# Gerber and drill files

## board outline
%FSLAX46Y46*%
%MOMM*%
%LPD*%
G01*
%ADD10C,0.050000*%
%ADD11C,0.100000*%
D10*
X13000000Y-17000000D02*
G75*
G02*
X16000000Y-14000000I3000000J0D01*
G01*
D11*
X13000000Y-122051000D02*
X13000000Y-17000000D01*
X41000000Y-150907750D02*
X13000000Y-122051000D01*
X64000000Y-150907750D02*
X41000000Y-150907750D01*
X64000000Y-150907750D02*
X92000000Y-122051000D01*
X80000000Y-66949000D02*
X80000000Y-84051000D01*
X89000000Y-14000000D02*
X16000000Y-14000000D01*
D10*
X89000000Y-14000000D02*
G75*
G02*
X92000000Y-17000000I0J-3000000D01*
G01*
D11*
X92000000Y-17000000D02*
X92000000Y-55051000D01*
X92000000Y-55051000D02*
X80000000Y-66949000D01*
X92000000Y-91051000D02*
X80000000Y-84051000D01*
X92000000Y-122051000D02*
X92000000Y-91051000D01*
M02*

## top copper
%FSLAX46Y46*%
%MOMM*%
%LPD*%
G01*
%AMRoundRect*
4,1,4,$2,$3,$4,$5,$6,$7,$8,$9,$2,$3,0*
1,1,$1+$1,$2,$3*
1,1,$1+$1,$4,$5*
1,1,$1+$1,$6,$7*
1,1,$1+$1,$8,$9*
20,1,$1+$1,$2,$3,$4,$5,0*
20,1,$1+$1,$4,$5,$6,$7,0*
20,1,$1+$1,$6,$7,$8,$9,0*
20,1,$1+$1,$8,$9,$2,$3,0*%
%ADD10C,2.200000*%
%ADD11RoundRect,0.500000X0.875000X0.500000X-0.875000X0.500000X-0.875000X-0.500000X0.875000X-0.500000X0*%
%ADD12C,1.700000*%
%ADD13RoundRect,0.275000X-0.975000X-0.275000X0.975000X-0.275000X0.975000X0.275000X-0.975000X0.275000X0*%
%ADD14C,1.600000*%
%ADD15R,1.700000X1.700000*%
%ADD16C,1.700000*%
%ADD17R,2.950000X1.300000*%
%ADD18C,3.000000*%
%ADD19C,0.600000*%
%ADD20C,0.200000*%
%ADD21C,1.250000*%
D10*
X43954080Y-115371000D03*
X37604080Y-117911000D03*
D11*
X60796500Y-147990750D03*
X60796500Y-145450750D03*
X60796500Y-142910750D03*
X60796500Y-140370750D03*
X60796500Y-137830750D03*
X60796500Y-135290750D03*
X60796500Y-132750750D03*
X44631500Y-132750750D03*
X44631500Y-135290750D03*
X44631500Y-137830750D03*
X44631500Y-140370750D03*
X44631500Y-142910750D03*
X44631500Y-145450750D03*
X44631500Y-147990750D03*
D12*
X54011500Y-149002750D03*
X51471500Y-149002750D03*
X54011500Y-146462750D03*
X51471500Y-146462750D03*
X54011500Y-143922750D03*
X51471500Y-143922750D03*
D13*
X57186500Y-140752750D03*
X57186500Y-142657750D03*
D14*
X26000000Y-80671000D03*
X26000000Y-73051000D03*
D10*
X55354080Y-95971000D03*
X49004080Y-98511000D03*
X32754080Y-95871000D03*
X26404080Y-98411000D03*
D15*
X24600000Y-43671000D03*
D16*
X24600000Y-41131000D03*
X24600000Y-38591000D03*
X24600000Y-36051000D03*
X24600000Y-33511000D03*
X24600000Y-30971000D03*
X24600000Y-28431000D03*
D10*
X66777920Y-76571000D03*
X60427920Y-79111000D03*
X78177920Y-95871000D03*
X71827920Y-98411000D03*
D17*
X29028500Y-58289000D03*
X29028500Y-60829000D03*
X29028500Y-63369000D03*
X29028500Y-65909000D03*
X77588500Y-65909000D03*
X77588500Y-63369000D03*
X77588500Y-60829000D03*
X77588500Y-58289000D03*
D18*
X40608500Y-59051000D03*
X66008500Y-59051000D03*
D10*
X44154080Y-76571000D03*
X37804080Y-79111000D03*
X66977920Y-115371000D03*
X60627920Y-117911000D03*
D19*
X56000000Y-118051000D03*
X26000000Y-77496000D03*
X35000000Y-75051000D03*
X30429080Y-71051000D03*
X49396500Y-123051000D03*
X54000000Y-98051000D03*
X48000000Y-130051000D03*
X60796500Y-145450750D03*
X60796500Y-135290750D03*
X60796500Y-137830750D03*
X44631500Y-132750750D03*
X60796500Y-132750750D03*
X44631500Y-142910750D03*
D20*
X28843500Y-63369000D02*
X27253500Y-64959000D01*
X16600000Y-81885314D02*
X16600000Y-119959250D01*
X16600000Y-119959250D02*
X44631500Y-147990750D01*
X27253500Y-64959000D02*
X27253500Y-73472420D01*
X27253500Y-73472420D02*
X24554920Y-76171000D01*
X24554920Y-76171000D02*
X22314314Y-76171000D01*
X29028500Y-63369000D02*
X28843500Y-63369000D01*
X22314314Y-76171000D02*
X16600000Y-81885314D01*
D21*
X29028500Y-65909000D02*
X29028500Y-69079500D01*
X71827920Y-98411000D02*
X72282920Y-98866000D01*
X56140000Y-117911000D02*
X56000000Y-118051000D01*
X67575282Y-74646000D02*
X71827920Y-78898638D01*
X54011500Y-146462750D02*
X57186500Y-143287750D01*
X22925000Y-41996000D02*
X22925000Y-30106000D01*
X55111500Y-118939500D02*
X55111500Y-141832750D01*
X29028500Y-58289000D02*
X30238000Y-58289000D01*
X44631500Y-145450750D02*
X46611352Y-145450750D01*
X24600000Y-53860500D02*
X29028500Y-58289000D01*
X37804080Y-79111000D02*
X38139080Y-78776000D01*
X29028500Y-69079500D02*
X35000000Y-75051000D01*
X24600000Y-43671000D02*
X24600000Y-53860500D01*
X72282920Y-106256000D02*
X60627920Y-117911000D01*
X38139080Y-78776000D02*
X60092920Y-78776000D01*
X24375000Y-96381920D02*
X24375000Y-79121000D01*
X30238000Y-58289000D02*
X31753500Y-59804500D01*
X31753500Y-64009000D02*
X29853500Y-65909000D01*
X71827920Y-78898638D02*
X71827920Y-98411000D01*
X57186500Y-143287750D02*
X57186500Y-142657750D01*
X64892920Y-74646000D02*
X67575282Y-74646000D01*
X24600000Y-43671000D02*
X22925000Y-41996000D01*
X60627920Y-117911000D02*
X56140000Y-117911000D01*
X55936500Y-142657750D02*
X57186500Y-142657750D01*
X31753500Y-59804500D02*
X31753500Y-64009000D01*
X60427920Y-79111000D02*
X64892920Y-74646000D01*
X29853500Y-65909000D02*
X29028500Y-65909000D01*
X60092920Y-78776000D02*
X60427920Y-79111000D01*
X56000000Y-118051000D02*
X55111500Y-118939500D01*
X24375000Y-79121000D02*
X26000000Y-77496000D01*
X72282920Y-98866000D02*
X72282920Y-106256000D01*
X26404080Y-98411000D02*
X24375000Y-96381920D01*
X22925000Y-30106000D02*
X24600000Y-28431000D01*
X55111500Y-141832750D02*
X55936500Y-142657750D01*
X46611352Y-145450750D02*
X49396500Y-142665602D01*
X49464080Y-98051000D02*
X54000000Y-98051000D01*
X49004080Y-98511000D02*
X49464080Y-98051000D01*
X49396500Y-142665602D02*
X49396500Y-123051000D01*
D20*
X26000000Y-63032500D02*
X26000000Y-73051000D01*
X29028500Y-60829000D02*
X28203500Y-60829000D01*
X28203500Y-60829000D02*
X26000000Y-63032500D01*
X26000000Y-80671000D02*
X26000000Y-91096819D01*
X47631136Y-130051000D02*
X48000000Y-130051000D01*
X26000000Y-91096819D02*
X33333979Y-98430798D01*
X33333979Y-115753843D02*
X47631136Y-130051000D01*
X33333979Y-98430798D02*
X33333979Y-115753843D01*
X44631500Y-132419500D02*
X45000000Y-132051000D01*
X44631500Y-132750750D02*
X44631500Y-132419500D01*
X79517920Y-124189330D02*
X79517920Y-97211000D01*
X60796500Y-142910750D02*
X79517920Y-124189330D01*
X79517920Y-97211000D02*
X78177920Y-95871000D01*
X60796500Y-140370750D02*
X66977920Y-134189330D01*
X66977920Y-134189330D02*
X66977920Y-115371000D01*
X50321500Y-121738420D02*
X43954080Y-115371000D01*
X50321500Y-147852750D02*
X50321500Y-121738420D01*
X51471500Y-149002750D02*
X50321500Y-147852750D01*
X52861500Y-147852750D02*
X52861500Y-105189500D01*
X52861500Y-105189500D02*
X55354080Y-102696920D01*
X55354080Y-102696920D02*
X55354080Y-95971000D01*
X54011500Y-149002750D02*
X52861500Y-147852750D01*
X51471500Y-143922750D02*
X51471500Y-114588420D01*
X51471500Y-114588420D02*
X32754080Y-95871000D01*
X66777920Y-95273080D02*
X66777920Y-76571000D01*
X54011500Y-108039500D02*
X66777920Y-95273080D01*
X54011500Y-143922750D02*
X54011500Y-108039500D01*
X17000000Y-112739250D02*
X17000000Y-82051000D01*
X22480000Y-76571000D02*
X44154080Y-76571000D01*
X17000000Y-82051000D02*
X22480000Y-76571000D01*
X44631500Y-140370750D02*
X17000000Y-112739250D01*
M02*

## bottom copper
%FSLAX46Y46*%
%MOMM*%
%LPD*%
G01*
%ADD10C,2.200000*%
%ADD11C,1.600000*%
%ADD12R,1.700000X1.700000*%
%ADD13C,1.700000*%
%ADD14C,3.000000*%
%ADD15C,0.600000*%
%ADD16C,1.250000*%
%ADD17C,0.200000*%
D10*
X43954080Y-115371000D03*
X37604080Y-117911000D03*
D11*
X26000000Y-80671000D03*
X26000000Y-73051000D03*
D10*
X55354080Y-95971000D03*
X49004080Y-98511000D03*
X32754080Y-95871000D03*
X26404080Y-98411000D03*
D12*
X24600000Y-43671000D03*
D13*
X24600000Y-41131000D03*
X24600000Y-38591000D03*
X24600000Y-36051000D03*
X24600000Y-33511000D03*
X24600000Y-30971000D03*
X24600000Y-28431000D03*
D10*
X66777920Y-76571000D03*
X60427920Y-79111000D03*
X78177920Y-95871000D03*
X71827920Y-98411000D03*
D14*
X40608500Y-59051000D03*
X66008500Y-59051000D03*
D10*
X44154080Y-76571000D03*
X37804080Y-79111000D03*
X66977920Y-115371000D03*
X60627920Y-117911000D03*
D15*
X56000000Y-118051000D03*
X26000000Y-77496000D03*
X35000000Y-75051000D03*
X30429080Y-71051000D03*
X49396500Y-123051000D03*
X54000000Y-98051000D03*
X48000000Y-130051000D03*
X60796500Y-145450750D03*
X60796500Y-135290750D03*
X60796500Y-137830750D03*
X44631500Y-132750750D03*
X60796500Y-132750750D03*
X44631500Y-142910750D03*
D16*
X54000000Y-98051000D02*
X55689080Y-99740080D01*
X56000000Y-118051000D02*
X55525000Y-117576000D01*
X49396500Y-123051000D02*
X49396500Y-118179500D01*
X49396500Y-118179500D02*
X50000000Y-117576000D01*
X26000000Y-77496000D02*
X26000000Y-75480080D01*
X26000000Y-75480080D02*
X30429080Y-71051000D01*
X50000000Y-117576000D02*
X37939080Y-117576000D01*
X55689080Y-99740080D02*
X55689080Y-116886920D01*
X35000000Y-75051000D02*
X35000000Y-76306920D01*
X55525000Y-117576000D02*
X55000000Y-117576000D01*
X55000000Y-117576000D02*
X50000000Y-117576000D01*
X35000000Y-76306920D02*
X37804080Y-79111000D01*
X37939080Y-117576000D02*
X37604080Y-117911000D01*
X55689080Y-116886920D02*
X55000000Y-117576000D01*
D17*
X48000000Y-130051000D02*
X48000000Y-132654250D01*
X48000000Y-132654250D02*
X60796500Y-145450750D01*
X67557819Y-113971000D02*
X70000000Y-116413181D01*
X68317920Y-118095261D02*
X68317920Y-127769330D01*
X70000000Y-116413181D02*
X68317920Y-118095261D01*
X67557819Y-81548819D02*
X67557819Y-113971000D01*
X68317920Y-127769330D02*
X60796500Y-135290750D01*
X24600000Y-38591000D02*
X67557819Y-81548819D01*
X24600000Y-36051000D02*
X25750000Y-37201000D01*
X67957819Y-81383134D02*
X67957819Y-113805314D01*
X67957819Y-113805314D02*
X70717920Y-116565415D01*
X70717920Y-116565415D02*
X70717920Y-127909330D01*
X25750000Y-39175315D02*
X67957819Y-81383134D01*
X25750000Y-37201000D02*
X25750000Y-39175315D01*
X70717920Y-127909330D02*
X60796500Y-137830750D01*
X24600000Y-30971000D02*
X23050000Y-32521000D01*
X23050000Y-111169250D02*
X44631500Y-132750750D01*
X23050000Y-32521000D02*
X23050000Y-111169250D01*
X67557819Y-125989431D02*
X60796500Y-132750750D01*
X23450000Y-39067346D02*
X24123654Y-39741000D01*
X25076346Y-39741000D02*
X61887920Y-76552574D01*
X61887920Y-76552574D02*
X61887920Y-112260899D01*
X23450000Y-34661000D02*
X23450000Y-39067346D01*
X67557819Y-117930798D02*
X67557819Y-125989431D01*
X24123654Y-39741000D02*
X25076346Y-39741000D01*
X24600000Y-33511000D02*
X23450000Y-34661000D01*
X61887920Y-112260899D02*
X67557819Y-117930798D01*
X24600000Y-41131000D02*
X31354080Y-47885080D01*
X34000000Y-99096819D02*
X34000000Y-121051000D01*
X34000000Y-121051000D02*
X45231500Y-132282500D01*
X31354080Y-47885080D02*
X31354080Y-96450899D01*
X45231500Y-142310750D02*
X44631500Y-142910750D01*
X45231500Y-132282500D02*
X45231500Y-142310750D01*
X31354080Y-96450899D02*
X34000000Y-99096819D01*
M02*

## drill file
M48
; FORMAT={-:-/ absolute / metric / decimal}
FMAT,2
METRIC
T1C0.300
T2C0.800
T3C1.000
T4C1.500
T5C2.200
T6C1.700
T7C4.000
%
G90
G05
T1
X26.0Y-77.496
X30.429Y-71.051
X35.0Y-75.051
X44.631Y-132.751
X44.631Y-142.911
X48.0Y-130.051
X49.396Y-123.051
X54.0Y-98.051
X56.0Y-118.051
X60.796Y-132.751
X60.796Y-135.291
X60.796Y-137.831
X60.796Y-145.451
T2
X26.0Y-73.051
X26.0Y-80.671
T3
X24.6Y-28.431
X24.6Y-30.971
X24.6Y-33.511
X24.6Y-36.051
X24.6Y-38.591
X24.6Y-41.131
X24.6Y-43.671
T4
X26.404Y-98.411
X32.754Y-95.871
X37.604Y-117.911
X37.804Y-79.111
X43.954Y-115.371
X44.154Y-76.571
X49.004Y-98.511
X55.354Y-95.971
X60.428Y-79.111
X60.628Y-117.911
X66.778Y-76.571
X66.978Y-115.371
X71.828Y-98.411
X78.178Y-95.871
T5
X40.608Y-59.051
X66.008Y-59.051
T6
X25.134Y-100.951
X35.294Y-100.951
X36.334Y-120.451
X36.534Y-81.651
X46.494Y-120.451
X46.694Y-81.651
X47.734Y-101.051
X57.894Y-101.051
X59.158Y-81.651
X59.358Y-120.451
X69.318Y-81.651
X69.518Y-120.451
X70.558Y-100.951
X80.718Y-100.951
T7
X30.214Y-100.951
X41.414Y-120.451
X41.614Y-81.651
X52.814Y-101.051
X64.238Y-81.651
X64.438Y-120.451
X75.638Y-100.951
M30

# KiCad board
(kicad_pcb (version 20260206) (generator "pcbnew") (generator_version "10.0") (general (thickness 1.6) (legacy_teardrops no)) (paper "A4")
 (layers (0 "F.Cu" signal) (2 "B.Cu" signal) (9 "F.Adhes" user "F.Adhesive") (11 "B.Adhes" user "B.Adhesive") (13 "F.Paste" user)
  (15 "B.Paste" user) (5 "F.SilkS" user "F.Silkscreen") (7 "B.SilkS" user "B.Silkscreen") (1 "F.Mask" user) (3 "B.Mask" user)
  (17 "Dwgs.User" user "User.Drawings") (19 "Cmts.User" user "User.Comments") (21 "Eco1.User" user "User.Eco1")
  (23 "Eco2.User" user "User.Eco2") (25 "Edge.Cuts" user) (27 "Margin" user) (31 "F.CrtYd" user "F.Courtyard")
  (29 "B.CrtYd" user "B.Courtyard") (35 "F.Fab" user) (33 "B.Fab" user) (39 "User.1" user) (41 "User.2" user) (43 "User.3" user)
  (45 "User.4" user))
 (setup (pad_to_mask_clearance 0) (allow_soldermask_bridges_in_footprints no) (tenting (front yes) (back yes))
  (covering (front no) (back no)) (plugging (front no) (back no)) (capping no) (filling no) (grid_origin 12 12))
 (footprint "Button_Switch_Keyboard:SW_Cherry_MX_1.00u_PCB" (layer "F.Cu") (at 43.95408 115.371)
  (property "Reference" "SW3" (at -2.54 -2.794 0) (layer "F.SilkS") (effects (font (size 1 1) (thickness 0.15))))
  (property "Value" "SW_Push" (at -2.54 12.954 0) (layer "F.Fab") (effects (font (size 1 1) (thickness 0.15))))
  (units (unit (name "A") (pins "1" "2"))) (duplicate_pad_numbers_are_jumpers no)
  (pad "" np_thru_hole circle (at -7.62 5.08) (size 1.7 1.7) (drill 1.7) (layers "*.Cu" "*.Mask"))
  (pad "" np_thru_hole circle (at -2.54 5.08) (size 4 4) (drill 4) (layers "*.Cu" "*.Mask"))
  (pad "" np_thru_hole circle (at 2.54 5.08) (size 1.7 1.7) (drill 1.7) (layers "*.Cu" "*.Mask"))
  (pad "1" thru_hole circle (at 0 0) (size 2.2 2.2) (drill 1.5) (layers "*.Cu" "*.Mask") (remove_unused_layers no) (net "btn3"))
  (pad "2" thru_hole circle (at -6.35 2.54) (size 2.2 2.2) (drill 1.5) (layers "*.Cu" "*.Mask") (remove_unused_layers no) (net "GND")))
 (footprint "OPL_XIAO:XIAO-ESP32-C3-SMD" (layer "F.Cu") (at 61.6315 129.87075 180)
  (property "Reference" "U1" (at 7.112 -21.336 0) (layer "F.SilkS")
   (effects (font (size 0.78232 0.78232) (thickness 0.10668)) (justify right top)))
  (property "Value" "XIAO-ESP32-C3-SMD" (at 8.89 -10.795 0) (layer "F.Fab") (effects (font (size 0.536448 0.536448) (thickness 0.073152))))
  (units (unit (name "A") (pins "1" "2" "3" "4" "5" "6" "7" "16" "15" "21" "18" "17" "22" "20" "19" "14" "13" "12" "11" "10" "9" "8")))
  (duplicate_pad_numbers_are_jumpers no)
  (pad "1" smd roundrect (at 0.835 -18.12 180) (size 2.75 2) (layers "F.Cu" "F.Mask" "F.Paste") (roundrect_rratio 0.25)
   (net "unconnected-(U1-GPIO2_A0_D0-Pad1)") (solder_mask_margin 0.0508) (thermal_bridge_angle 45))
  (pad "2" smd roundrect (at 0.835 -15.58 180) (size 2.75 2) (layers "F.Cu" "F.Mask" "F.Paste") (roundrect_rratio 0.25) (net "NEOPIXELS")
   (solder_mask_margin 0.0508) (thermal_bridge_angle 45))
  (pad "3" smd roundrect (at 0.835 -13.04 180) (size 2.75 2) (layers "F.Cu" "F.Mask" "F.Paste") (roundrect_rratio 0.25) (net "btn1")
   (solder_mask_margin 0.0508) (thermal_bridge_angle 45))
  (pad "4" smd roundrect (at 0.835 -10.5 180) (size 2.75 2) (layers "F.Cu" "F.Mask" "F.Paste") (roundrect_rratio 0.25) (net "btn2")
   (solder_mask_margin 0.0508) (thermal_bridge_angle 45))
  (pad "5" smd roundrect (at 0.835 -7.96 180) (size 2.75 2) (layers "F.Cu" "F.Mask" "F.Paste") (roundrect_rratio 0.25) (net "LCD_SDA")
   (solder_mask_margin 0.0508) (thermal_bridge_angle 45))
  (pad "6" smd roundrect (at 0.835 -5.42 180) (size 2.75 2) (layers "F.Cu" "F.Mask" "F.Paste") (roundrect_rratio 0.25) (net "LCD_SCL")
   (solder_mask_margin 0.0508) (thermal_bridge_angle 45))
  (pad "7" smd roundrect (at 0.835 -2.88 180) (size 2.75 2) (layers "F.Cu" "F.Mask" "F.Paste") (roundrect_rratio 0.25) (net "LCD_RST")
   (solder_mask_margin 0.0508) (thermal_bridge_angle 45))
  (pad "8" smd roundrect (at 17 -2.88 180) (size 2.75 2) (layers "F.Cu" "F.Mask" "F.Paste") (roundrect_rratio 0.25) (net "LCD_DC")
   (solder_mask_margin 0.0508) (thermal_bridge_angle 45))
  (pad "9" smd roundrect (at 17 -5.42 180) (size 2.75 2) (layers "F.Cu" "F.Mask" "F.Paste") (roundrect_rratio 0.25)
   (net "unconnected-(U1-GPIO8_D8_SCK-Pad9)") (solder_mask_margin 0.0508) (thermal_bridge_angle 45))
  (pad "10" smd roundrect (at 17 -7.96 180) (size 2.75 2) (layers "F.Cu" "F.Mask" "F.Paste") (roundrect_rratio 0.25)
   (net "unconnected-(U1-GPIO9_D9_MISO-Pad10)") (solder_mask_margin 0.0508) (thermal_bridge_angle 45))
  (pad "11" smd roundrect (at 17 -10.5 180) (size 2.75 2) (layers "F.Cu" "F.Mask" "F.Paste") (roundrect_rratio 0.25) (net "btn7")
   (solder_mask_margin 0.0508) (thermal_bridge_angle 45))
  (pad "12" smd roundrect (at 17 -13.04 180) (size 2.75 2) (layers "F.Cu" "F.Mask" "F.Paste") (roundrect_rratio 0.25) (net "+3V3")
   (solder_mask_margin 0.0508) (thermal_bridge_angle 45))
  (pad "13" smd roundrect (at 17 -15.58 180) (size 2.75 2) (layers "F.Cu" "F.Mask" "F.Paste") (roundrect_rratio 0.25) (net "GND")
   (solder_mask_margin 0.0508) (thermal_bridge_angle 45))
  (pad "14" smd roundrect (at 17 -18.12 180) (size 2.75 2) (layers "F.Cu" "F.Mask" "F.Paste") (roundrect_rratio 0.25) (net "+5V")
   (solder_mask_margin 0.0508) (thermal_bridge_angle 45))
  (pad "15" smd circle (at 7.62 -19.132 180) (size 1.7 1.7) (layers "F.Cu" "F.Mask" "F.Paste") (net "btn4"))
  (pad "16" smd circle (at 10.16 -19.132 180) (size 1.7 1.7) (layers "F.Cu" "F.Mask" "F.Paste") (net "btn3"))
  (pad "17" smd circle (at 7.62 -16.592 180) (size 1.7 1.7) (layers "F.Cu" "F.Mask" "F.Paste") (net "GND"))
  (pad "18" smd circle (at 10.16 -16.592 180) (size 1.7 1.7) (layers "F.Cu" "F.Mask" "F.Paste") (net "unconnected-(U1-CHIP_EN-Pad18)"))
  (pad "19" smd circle (at 7.62 -14.052 180) (size 1.7 1.7) (layers "F.Cu" "F.Mask" "F.Paste") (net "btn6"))
  (pad "20" smd circle (at 10.16 -14.052 180) (size 1.7 1.7) (layers "F.Cu" "F.Mask" "F.Paste") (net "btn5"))
  (pad "21" smd roundrect (at 4.445 -10.882) (size 2.5 1.1) (layers "F.Cu" "F.Mask" "F.Paste") (roundrect_rratio 0.25) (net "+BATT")
   (thermal_bridge_angle 45))
  (pad "22" smd roundrect (at 4.445 -12.787) (size 2.5 1.1) (layers "F.Cu" "F.Mask" "F.Paste") (roundrect_rratio 0.25) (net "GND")
   (thermal_bridge_angle 45)))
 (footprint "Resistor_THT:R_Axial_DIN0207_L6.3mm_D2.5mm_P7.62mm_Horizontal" (layer "F.Cu") (at 26 80.671 90)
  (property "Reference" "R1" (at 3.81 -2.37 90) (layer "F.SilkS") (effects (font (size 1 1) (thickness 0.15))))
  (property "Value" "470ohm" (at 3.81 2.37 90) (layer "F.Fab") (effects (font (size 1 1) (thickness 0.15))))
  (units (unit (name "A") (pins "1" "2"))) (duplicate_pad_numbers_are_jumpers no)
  (pad "1" thru_hole circle (at 0 0 90) (size 1.6 1.6) (drill 0.8) (layers "*.Cu" "*.Mask") (remove_unused_layers no) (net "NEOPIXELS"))
  (pad "2" thru_hole circle (at 7.62 0 90) (size 1.6 1.6) (drill 0.8) (layers "*.Cu" "*.Mask") (remove_unused_layers no)
   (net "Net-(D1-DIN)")))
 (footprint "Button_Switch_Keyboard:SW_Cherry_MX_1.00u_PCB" (layer "F.Cu") (at 55.35408 95.971)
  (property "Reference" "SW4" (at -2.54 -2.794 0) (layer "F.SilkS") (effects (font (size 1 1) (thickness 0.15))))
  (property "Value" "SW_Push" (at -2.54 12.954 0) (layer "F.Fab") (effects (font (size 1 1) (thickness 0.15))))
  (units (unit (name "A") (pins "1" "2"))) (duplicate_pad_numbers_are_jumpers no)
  (pad "" np_thru_hole circle (at -7.62 5.08) (size 1.7 1.7) (drill 1.7) (layers "*.Cu" "*.Mask"))
  (pad "" np_thru_hole circle (at -2.54 5.08) (size 4 4) (drill 4) (layers "*.Cu" "*.Mask"))
  (pad "" np_thru_hole circle (at 2.54 5.08) (size 1.7 1.7) (drill 1.7) (layers "*.Cu" "*.Mask"))
  (pad "1" thru_hole circle (at 0 0) (size 2.2 2.2) (drill 1.5) (layers "*.Cu" "*.Mask") (remove_unused_layers no) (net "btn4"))
  (pad "2" thru_hole circle (at -6.35 2.54) (size 2.2 2.2) (drill 1.5) (layers "*.Cu" "*.Mask") (remove_unused_layers no) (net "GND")))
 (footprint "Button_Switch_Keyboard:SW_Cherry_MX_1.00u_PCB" (layer "F.Cu") (at 32.75408 95.871)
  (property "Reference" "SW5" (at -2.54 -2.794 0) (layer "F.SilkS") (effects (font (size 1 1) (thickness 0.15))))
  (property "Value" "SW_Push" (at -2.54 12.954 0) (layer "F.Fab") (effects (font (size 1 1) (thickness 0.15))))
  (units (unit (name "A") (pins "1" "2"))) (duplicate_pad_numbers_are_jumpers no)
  (pad "" np_thru_hole circle (at -7.62 5.08) (size 1.7 1.7) (drill 1.7) (layers "*.Cu" "*.Mask"))
  (pad "" np_thru_hole circle (at -2.54 5.08) (size 4 4) (drill 4) (layers "*.Cu" "*.Mask"))
  (pad "" np_thru_hole circle (at 2.54 5.08) (size 1.7 1.7) (drill 1.7) (layers "*.Cu" "*.Mask"))
  (pad "1" thru_hole circle (at 0 0) (size 2.2 2.2) (drill 1.5) (layers "*.Cu" "*.Mask") (remove_unused_layers no) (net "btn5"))
  (pad "2" thru_hole circle (at -6.35 2.54) (size 2.2 2.2) (drill 1.5) (layers "*.Cu" "*.Mask") (remove_unused_layers no) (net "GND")))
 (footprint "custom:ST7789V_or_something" (layer "F.Cu") (at 24.6 43.671 90)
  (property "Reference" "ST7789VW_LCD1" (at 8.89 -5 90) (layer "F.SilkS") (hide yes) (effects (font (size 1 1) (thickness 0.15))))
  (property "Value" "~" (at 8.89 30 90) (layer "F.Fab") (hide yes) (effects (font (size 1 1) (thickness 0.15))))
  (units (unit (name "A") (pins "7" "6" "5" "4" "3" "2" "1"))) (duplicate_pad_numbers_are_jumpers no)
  (pad "1" thru_hole rect (at 0 0 90) (size 1.7 1.7) (drill 1) (layers "*.Cu" "*.Mask") (remove_unused_layers no) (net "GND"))
  (pad "2" thru_hole circle (at 2.54 0 90) (size 1.7 1.7) (drill 1) (layers "*.Cu" "*.Mask") (remove_unused_layers no) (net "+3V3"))
  (pad "3" thru_hole circle (at 5.08 0 90) (size 1.7 1.7) (drill 1) (layers "*.Cu" "*.Mask") (remove_unused_layers no) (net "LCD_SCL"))
  (pad "4" thru_hole circle (at 7.62 0 90) (size 1.7 1.7) (drill 1) (layers "*.Cu" "*.Mask") (remove_unused_layers no) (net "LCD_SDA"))
  (pad "5" thru_hole circle (at 10.16 0 90) (size 1.7 1.7) (drill 1) (layers "*.Cu" "*.Mask") (remove_unused_layers no) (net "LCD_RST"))
  (pad "6" thru_hole circle (at 12.7 0 90) (size 1.7 1.7) (drill 1) (layers "*.Cu" "*.Mask") (remove_unused_layers no) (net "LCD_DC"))
  (pad "7" thru_hole circle (at 15.24 0 90) (size 1.7 1.7) (drill 1) (layers "*.Cu" "*.Mask") (remove_unused_layers no) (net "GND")))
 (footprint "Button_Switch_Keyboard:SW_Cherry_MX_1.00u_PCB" (layer "F.Cu") (at 66.77792 76.571)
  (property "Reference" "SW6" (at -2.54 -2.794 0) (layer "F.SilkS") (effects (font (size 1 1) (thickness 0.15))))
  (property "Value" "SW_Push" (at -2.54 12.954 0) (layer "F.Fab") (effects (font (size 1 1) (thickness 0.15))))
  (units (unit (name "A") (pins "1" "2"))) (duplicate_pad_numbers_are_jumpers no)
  (pad "" np_thru_hole circle (at -7.62 5.08) (size 1.7 1.7) (drill 1.7) (layers "*.Cu" "*.Mask"))
  (pad "" np_thru_hole circle (at -2.54 5.08) (size 4 4) (drill 4) (layers "*.Cu" "*.Mask"))
  (pad "" np_thru_hole circle (at 2.54 5.08) (size 1.7 1.7) (drill 1.7) (layers "*.Cu" "*.Mask"))
  (pad "1" thru_hole circle (at 0 0) (size 2.2 2.2) (drill 1.5) (layers "*.Cu" "*.Mask") (remove_unused_layers no) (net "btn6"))
  (pad "2" thru_hole circle (at -6.35 2.54) (size 2.2 2.2) (drill 1.5) (layers "*.Cu" "*.Mask") (remove_unused_layers no) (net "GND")))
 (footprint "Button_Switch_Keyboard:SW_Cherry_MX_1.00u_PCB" (layer "F.Cu") (at 78.17792 95.871)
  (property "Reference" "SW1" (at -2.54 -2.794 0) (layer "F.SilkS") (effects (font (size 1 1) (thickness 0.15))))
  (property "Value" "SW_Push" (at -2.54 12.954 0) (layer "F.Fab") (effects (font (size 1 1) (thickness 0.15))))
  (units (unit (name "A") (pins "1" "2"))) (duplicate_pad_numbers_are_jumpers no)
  (pad "" np_thru_hole circle (at -7.62 5.08) (size 1.7 1.7) (drill 1.7) (layers "*.Cu" "*.Mask"))
  (pad "" np_thru_hole circle (at -2.54 5.08) (size 4 4) (drill 4) (layers "*.Cu" "*.Mask"))
  (pad "" np_thru_hole circle (at 2.54 5.08) (size 1.7 1.7) (drill 1.7) (layers "*.Cu" "*.Mask"))
  (pad "1" thru_hole circle (at 0 0) (size 2.2 2.2) (drill 1.5) (layers "*.Cu" "*.Mask") (remove_unused_layers no) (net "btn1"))
  (pad "2" thru_hole circle (at -6.35 2.54) (size 2.2 2.2) (drill 1.5) (layers "*.Cu" "*.Mask") (remove_unused_layers no) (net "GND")))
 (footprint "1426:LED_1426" (layer "F.Cu") (at 53.3085 62.099)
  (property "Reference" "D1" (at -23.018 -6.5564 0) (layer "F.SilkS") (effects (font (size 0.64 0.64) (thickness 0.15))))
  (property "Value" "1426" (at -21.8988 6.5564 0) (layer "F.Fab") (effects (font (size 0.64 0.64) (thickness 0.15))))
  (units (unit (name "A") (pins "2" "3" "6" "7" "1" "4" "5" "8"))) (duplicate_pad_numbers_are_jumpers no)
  (pad "1" smd rect (at -24.28 -3.81) (size 2.95 1.3) (layers "F.Cu" "F.Mask" "F.Paste") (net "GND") (solder_mask_margin 0.102))
  (pad "2" smd rect (at -24.28 -1.27) (size 2.95 1.3) (layers "F.Cu" "F.Mask" "F.Paste") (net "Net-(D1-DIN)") (solder_mask_margin 0.102))
  (pad "3" smd rect (at -24.28 1.27) (size 2.95 1.3) (layers "F.Cu" "F.Mask" "F.Paste") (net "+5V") (solder_mask_margin 0.102))
  (pad "4" smd rect (at -24.28 3.81) (size 2.95 1.3) (layers "F.Cu" "F.Mask" "F.Paste") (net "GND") (solder_mask_margin 0.102))
  (pad "5" smd rect (at 24.28 3.81) (size 2.95 1.3) (layers "F.Cu" "F.Mask" "F.Paste") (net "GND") (solder_mask_margin 0.102))
  (pad "6" smd rect (at 24.28 1.27) (size 2.95 1.3) (layers "F.Cu" "F.Mask" "F.Paste") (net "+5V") (solder_mask_margin 0.102))
  (pad "7" smd rect (at 24.28 -1.27) (size 2.95 1.3) (layers "F.Cu" "F.Mask" "F.Paste") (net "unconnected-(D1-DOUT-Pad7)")
   (solder_mask_margin 0.102))
  (pad "8" smd rect (at 24.28 -3.81) (size 2.95 1.3) (layers "F.Cu" "F.Mask" "F.Paste") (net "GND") (solder_mask_margin 0.102))
  (pad "SH1" thru_hole circle (at -12.7 -3.048) (size 3 3) (drill 2.2) (layers "*.Cu" "*.Mask") (remove_unused_layers no)
   (solder_mask_margin 0.102))
  (pad "SH2" thru_hole circle (at 12.7 -3.048) (size 3 3) (drill 2.2) (layers "*.Cu" "*.Mask") (remove_unused_layers no)
   (solder_mask_margin 0.102)))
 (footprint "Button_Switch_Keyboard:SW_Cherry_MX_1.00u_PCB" (layer "F.Cu") (at 44.15408 76.571)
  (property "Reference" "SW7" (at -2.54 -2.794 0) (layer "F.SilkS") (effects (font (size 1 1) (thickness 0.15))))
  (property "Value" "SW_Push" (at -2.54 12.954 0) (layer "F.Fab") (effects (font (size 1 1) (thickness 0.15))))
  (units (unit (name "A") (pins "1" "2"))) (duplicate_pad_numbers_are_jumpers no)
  (pad "" np_thru_hole circle (at -7.62 5.08) (size 1.7 1.7) (drill 1.7) (layers "*.Cu" "*.Mask"))
  (pad "" np_thru_hole circle (at -2.54 5.08) (size 4 4) (drill 4) (layers "*.Cu" "*.Mask"))
  (pad "" np_thru_hole circle (at 2.54 5.08) (size 1.7 1.7) (drill 1.7) (layers "*.Cu" "*.Mask"))
  (pad "1" thru_hole circle (at 0 0) (size 2.2 2.2) (drill 1.5) (layers "*.Cu" "*.Mask") (remove_unused_layers no) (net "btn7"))
  (pad "2" thru_hole circle (at -6.35 2.54) (size 2.2 2.2) (drill 1.5) (layers "*.Cu" "*.Mask") (remove_unused_layers no) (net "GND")))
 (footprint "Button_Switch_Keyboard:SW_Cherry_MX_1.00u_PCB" (layer "F.Cu") (at 66.97792 115.371)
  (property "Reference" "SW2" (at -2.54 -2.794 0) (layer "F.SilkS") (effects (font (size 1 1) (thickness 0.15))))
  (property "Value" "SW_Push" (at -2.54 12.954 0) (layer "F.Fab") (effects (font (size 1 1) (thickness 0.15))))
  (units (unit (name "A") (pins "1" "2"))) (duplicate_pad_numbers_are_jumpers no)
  (pad "" np_thru_hole circle (at -7.62 5.08) (size 1.7 1.7) (drill 1.7) (layers "*.Cu" "*.Mask"))
  (pad "" np_thru_hole circle (at -2.54 5.08) (size 4 4) (drill 4) (layers "*.Cu" "*.Mask"))
  (pad "" np_thru_hole circle (at 2.54 5.08) (size 1.7 1.7) (drill 1.7) (layers "*.Cu" "*.Mask"))
  (pad "1" thru_hole circle (at 0 0) (size 2.2 2.2) (drill 1.5) (layers "*.Cu" "*.Mask") (remove_unused_layers no) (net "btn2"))
  (pad "2" thru_hole circle (at -6.35 2.54) (size 2.2 2.2) (drill 1.5) (layers "*.Cu" "*.Mask") (remove_unused_layers no) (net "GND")))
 (gr_arc (start 13 17) (mid 13.87868 14.87868) (end 16 14) (stroke (width 0.05) (type solid)) (layer "Edge.Cuts"))
 (gr_line (start 13 122.051) (end 13 17) (stroke (width 0.1) (type solid)) (layer "Edge.Cuts"))
 (gr_line (start 41 150.90775) (end 13 122.051) (stroke (width 0.1) (type solid)) (layer "Edge.Cuts"))
 (gr_line (start 64 150.90775) (end 41 150.90775) (stroke (width 0.1) (type solid)) (layer "Edge.Cuts"))
 (gr_line (start 64 150.90775) (end 92 122.051) (stroke (width 0.1) (type solid)) (layer "Edge.Cuts"))
 (gr_line (start 80 66.949) (end 80 84.051) (stroke (width 0.1) (type solid)) (layer "Edge.Cuts"))
 (gr_line (start 89 14) (end 16 14) (stroke (width 0.1) (type solid)) (layer "Edge.Cuts"))
 (gr_arc (start 89 14) (mid 91.12132 14.87868) (end 92 17) (stroke (width 0.05) (type default)) (layer "Edge.Cuts"))
 (gr_line (start 92 17) (end 92 55.051) (stroke (width 0.1) (type solid)) (layer "Edge.Cuts"))
 (gr_line (start 92 55.051) (end 80 66.949) (stroke (width 0.1) (type solid)) (layer "Edge.Cuts"))
 (gr_line (start 92 91.051) (end 80 84.051) (stroke (width 0.1) (type solid)) (layer "Edge.Cuts"))
 (gr_line (start 92 122.051) (end 92 91.051) (stroke (width 0.1) (type solid)) (layer "Edge.Cuts"))
 (segment (start 28.8435 63.369) (end 27.2535 64.959) (width 0.2) (layer "F.Cu") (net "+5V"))
 (segment (start 16.6 81.885314) (end 16.6 119.95925) (width 0.2) (layer "F.Cu") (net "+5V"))
 (segment (start 16.6 119.95925) (end 44.6315 147.99075) (width 0.2) (layer "F.Cu") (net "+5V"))
 (segment (start 27.2535 64.959) (end 27.2535 73.47242) (width 0.2) (layer "F.Cu") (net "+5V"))
 (segment (start 27.2535 73.47242) (end 24.55492 76.171) (width 0.2) (layer "F.Cu") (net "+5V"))
 (segment (start 24.55492 76.171) (end 22.314314 76.171) (width 0.2) (layer "F.Cu") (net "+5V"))
 (segment (start 29.0285 63.369) (end 28.8435 63.369) (width 0.2) (layer "F.Cu") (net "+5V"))
 (segment (start 22.314314 76.171) (end 16.6 81.885314) (width 0.2) (layer "F.Cu") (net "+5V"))
 (segment (start 29.0285 65.909) (end 29.0285 69.0795) (width 1.25) (layer "F.Cu") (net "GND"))
 (segment (start 71.82792 98.411) (end 72.28292 98.866) (width 1.25) (layer "F.Cu") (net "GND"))
 (segment (start 56.14 117.911) (end 56 118.051) (width 1.25) (layer "F.Cu") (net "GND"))
 (segment (start 67.575282 74.646) (end 71.82792 78.898638) (width 1.25) (layer "F.Cu") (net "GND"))
 (segment (start 54.0115 146.46275) (end 57.1865 143.28775) (width 1.25) (layer "F.Cu") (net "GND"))
 (segment (start 22.925 41.996) (end 22.925 30.106) (width 1.25) (layer "F.Cu") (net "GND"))
 (segment (start 55.1115 118.9395) (end 55.1115 141.83275) (width 1.25) (layer "F.Cu") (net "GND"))
 (segment (start 29.0285 58.289) (end 30.238 58.289) (width 1.25) (layer "F.Cu") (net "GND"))
 (segment (start 44.6315 145.45075) (end 46.611352 145.45075) (width 1.25) (layer "F.Cu") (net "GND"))
 (segment (start 24.6 53.8605) (end 29.0285 58.289) (width 1.25) (layer "F.Cu") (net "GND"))
 (segment (start 37.80408 79.111) (end 38.13908 78.776) (width 1.25) (layer "F.Cu") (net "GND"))
 (segment (start 29.0285 69.0795) (end 35 75.051) (width 1.25) (layer "F.Cu") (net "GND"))
 (segment (start 24.6 43.671) (end 24.6 53.8605) (width 1.25) (layer "F.Cu") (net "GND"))
 (segment (start 72.28292 106.256) (end 60.62792 117.911) (width 1.25) (layer "F.Cu") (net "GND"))
 (segment (start 38.13908 78.776) (end 60.09292 78.776) (width 1.25) (layer "F.Cu") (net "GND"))
 (segment (start 24.375 96.38192) (end 24.375 79.121) (width 1.25) (layer "F.Cu") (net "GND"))
 (segment (start 30.238 58.289) (end 31.7535 59.8045) (width 1.25) (layer "F.Cu") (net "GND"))
 (segment (start 31.7535 64.009) (end 29.8535 65.909) (width 1.25) (layer "F.Cu") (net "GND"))
 (segment (start 71.82792 78.898638) (end 71.82792 98.411) (width 1.25) (layer "F.Cu") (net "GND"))
 (segment (start 57.1865 143.28775) (end 57.1865 142.65775) (width 1.25) (layer "F.Cu") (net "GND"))
 (segment (start 64.89292 74.646) (end 67.575282 74.646) (width 1.25) (layer "F.Cu") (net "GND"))
 (segment (start 24.6 43.671) (end 22.925 41.996) (width 1.25) (layer "F.Cu") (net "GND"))
 (segment (start 60.62792 117.911) (end 56.14 117.911) (width 1.25) (layer "F.Cu") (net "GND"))
 (segment (start 55.9365 142.65775) (end 57.1865 142.65775) (width 1.25) (layer "F.Cu") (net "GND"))
 (segment (start 31.7535 59.8045) (end 31.7535 64.009) (width 1.25) (layer "F.Cu") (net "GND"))
 (segment (start 60.42792 79.111) (end 64.89292 74.646) (width 1.25) (layer "F.Cu") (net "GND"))
 (segment (start 29.8535 65.909) (end 29.0285 65.909) (width 1.25) (layer "F.Cu") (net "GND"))
 (segment (start 60.09292 78.776) (end 60.42792 79.111) (width 1.25) (layer "F.Cu") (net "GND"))
 (segment (start 56 118.051) (end 55.1115 118.9395) (width 1.25) (layer "F.Cu") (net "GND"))
 (segment (start 24.375 79.121) (end 26 77.496) (width 1.25) (layer "F.Cu") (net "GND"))
 (segment (start 72.28292 98.866) (end 72.28292 106.256) (width 1.25) (layer "F.Cu") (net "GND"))
 (segment (start 26.40408 98.411) (end 24.375 96.38192) (width 1.25) (layer "F.Cu") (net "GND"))
 (segment (start 22.925 30.106) (end 24.6 28.431) (width 1.25) (layer "F.Cu") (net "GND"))
 (segment (start 55.1115 141.83275) (end 55.9365 142.65775) (width 1.25) (layer "F.Cu") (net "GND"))
 (segment (start 46.611352 145.45075) (end 49.3965 142.665602) (width 1.25) (layer "F.Cu") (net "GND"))
 (segment (start 49.46408 98.051) (end 54 98.051) (width 1.25) (layer "F.Cu") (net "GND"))
 (segment (start 49.00408 98.511) (end 49.46408 98.051) (width 1.25) (layer "F.Cu") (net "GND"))
 (segment (start 49.3965 142.665602) (end 49.3965 123.051) (width 1.25) (layer "F.Cu") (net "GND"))
 (via (at 56 118.051) (size 0.6) (drill 0.3) (layers "F.Cu" "B.Cu") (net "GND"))
 (via (at 26 77.496) (size 0.6) (drill 0.3) (layers "F.Cu" "B.Cu") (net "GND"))
 (via (at 35 75.051) (size 0.6) (drill 0.3) (layers "F.Cu" "B.Cu") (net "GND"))
 (via (at 30.42908 71.051) (size 0.6) (drill 0.3) (layers "F.Cu" "B.Cu") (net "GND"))
 (via (at 49.3965 123.051) (size 0.6) (drill 0.3) (layers "F.Cu" "B.Cu") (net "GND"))
 (via (at 54 98.051) (size 0.6) (drill 0.3) (layers "F.Cu" "B.Cu") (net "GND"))
 (segment (start 54 98.051) (end 55.68908 99.74008) (width 1.25) (layer "B.Cu") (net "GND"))
 (segment (start 56 118.051) (end 55.525 117.576) (width 1.25) (layer "B.Cu") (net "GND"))
 (segment (start 49.3965 123.051) (end 49.3965 118.1795) (width 1.25) (layer "B.Cu") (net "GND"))
 (segment (start 49.3965 118.1795) (end 50 117.576) (width 1.25) (layer "B.Cu") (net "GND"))
 (segment (start 26 77.496) (end 26 75.48008) (width 1.25) (layer "B.Cu") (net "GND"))
 (segment (start 26 75.48008) (end 30.42908 71.051) (width 1.25) (layer "B.Cu") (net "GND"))
 (segment (start 50 117.576) (end 37.93908 117.576) (width 1.25) (layer "B.Cu") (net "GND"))
 (segment (start 55.68908 99.74008) (end 55.68908 116.88692) (width 1.25) (layer "B.Cu") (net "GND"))
 (segment (start 35 75.051) (end 35 76.30692) (width 1.25) (layer "B.Cu") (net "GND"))
 (segment (start 55.525 117.576) (end 55 117.576) (width 1.25) (layer "B.Cu") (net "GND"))
 (segment (start 55 117.576) (end 50 117.576) (width 1.25) (layer "B.Cu") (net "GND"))
 (segment (start 35 76.30692) (end 37.80408 79.111) (width 1.25) (layer "B.Cu") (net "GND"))
 (segment (start 37.93908 117.576) (end 37.60408 117.911) (width 1.25) (layer "B.Cu") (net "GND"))
 (segment (start 55.68908 116.88692) (end 55 117.576) (width 1.25) (layer "B.Cu") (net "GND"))
 (segment (start 26 63.0325) (end 26 73.051) (width 0.2) (layer "F.Cu") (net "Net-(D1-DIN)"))
 (segment (start 29.0285 60.829) (end 28.2035 60.829) (width 0.2) (layer "F.Cu") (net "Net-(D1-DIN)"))
 (segment (start 28.2035 60.829) (end 26 63.0325) (width 0.2) (layer "F.Cu") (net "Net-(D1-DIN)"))
 (segment (start 26 80.671) (end 26 91.096819) (width 0.2) (layer "F.Cu") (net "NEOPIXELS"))
 (segment (start 47.631136 130.051) (end 48 130.051) (width 0.2) (layer "F.Cu") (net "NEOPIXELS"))
 (segment (start 26 91.096819) (end 33.333979 98.430798) (width 0.2) (layer "F.Cu") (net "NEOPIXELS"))
 (segment (start 33.333979 115.753843) (end 47.631136 130.051) (width 0.2) (layer "F.Cu") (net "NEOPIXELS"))
 (segment (start 33.333979 98.430798) (end 33.333979 115.753843) (width 0.2) (layer "F.Cu") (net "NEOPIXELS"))
 (via (at 48 130.051) (size 0.6) (drill 0.3) (layers "F.Cu" "B.Cu") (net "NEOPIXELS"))
 (via (at 60.7965 145.45075) (size 0.6) (drill 0.3) (layers "F.Cu" "B.Cu") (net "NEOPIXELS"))
 (segment (start 48 130.051) (end 48 132.65425) (width 0.2) (layer "B.Cu") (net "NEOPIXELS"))
 (segment (start 48 132.65425) (end 60.7965 145.45075) (width 0.2) (layer "B.Cu") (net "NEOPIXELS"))
 (via (at 60.7965 135.29075) (size 0.6) (drill 0.3) (layers "F.Cu" "B.Cu") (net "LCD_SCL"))
 (segment (start 67.557819 113.971) (end 70 116.413181) (width 0.2) (layer "B.Cu") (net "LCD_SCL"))
 (segment (start 68.31792 118.095261) (end 68.31792 127.76933) (width 0.2) (layer "B.Cu") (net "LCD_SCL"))
 (segment (start 70 116.413181) (end 68.31792 118.095261) (width 0.2) (layer "B.Cu") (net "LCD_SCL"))
 (segment (start 67.557819 81.548819) (end 67.557819 113.971) (width 0.2) (layer "B.Cu") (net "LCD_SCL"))
 (segment (start 68.31792 127.76933) (end 60.7965 135.29075) (width 0.2) (layer "B.Cu") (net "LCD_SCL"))
 (segment (start 24.6 38.591) (end 67.557819 81.548819) (width 0.2) (layer "B.Cu") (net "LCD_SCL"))
 (via (at 60.7965 137.83075) (size 0.6) (drill 0.3) (layers "F.Cu" "B.Cu") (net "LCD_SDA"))
 (segment (start 24.6 36.051) (end 25.75 37.201) (width 0.2) (layer "B.Cu") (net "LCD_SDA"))
 (segment (start 67.957819 81.383134) (end 67.957819 113.805314) (width 0.2) (layer "B.Cu") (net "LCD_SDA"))
 (segment (start 67.957819 113.805314) (end 70.71792 116.565415) (width 0.2) (layer "B.Cu") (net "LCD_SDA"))
 (segment (start 70.71792 116.565415) (end 70.71792 127.90933) (width 0.2) (layer "B.Cu") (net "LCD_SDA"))
 (segment (start 25.75 39.175315) (end 67.957819 81.383134) (width 0.2) (layer "B.Cu") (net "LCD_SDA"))
 (segment (start 25.75 37.201) (end 25.75 39.175315) (width 0.2) (layer "B.Cu") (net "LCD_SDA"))
 (segment (start 70.71792 127.90933) (end 60.7965 137.83075) (width 0.2) (layer "B.Cu") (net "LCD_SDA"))
 (segment (start 44.6315 132.4195) (end 45 132.051) (width 0.2) (layer "F.Cu") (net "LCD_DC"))
 (segment (start 44.6315 132.75075) (end 44.6315 132.4195) (width 0.2) (layer "F.Cu") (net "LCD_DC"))
 (via (at 44.6315 132.75075) (size 0.6) (drill 0.3) (layers "F.Cu" "B.Cu") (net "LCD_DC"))
 (segment (start 24.6 30.971) (end 23.05 32.521) (width 0.2) (layer "B.Cu") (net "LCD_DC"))
 (segment (start 23.05 111.16925) (end 44.6315 132.75075) (width 0.2) (layer "B.Cu") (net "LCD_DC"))
 (segment (start 23.05 32.521) (end 23.05 111.16925) (width 0.2) (layer "B.Cu") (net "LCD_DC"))
 (via (at 60.7965 132.75075) (size 0.6) (drill 0.3) (layers "F.Cu" "B.Cu") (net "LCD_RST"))
 (segment (start 67.557819 125.989431) (end 60.7965 132.75075) (width 0.2) (layer "B.Cu") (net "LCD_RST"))
 (segment (start 23.45 39.067346) (end 24.123654 39.741) (width 0.2) (layer "B.Cu") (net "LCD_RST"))
 (segment (start 25.076346 39.741) (end 61.88792 76.552574) (width 0.2) (layer "B.Cu") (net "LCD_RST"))
 (segment (start 61.88792 76.552574) (end 61.88792 112.260899) (width 0.2) (layer "B.Cu") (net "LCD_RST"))
 (segment (start 23.45 34.661) (end 23.45 39.067346) (width 0.2) (layer "B.Cu") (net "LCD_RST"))
 (segment (start 67.557819 117.930798) (end 67.557819 125.989431) (width 0.2) (layer "B.Cu") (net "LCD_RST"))
 (segment (start 24.123654 39.741) (end 25.076346 39.741) (width 0.2) (layer "B.Cu") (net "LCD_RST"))
 (segment (start 24.6 33.511) (end 23.45 34.661) (width 0.2) (layer "B.Cu") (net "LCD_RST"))
 (segment (start 61.88792 112.260899) (end 67.557819 117.930798) (width 0.2) (layer "B.Cu") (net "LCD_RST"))
 (via (at 44.6315 142.91075) (size 0.6) (drill 0.3) (layers "F.Cu" "B.Cu") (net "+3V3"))
 (segment (start 24.6 41.131) (end 31.35408 47.88508) (width 0.2) (layer "B.Cu") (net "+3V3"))
 (segment (start 34 99.096819) (end 34 121.051) (width 0.2) (layer "B.Cu") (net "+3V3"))
 (segment (start 34 121.051) (end 45.2315 132.2825) (width 0.2) (layer "B.Cu") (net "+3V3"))
 (segment (start 31.35408 47.88508) (end 31.35408 96.450899) (width 0.2) (layer "B.Cu") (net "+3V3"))
 (segment (start 45.2315 142.31075) (end 44.6315 142.91075) (width 0.2) (layer "B.Cu") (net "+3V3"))
 (segment (start 45.2315 132.2825) (end 45.2315 142.31075) (width 0.2) (layer "B.Cu") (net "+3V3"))
 (segment (start 31.35408 96.450899) (end 34 99.096819) (width 0.2) (layer "B.Cu") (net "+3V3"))
 (segment (start 79.51792 124.18933) (end 79.51792 97.211) (width 0.2) (layer "F.Cu") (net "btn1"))
 (segment (start 60.7965 142.91075) (end 79.51792 124.18933) (width 0.2) (layer "F.Cu") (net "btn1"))
 (segment (start 79.51792 97.211) (end 78.17792 95.871) (width 0.2) (layer "F.Cu") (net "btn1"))
 (segment (start 60.7965 140.37075) (end 66.97792 134.18933) (width 0.2) (layer "F.Cu") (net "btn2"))
 (segment (start 66.97792 134.18933) (end 66.97792 115.371) (width 0.2) (layer "F.Cu") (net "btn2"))
 (segment (start 50.3215 121.73842) (end 43.95408 115.371) (width 0.2) (layer "F.Cu") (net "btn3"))
 (segment (start 50.3215 147.85275) (end 50.3215 121.73842) (width 0.2) (layer "F.Cu") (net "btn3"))
 (segment (start 51.4715 149.00275) (end 50.3215 147.85275) (width 0.2) (layer "F.Cu") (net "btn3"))
 (segment (start 52.8615 147.85275) (end 52.8615 105.1895) (width 0.2) (layer "F.Cu") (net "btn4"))
 (segment (start 52.8615 105.1895) (end 55.35408 102.69692) (width 0.2) (layer "F.Cu") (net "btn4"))
 (segment (start 55.35408 102.69692) (end 55.35408 95.971) (width 0.2) (layer "F.Cu") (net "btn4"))
 (segment (start 54.0115 149.00275) (end 52.8615 147.85275) (width 0.2) (layer "F.Cu") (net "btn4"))
 (segment (start 51.4715 143.92275) (end 51.4715 114.58842) (width 0.2) (layer "F.Cu") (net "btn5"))
 (segment (start 51.4715 114.58842) (end 32.75408 95.871) (width 0.2) (layer "F.Cu") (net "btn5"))
 (segment (start 66.77792 95.27308) (end 66.77792 76.571) (width 0.2) (layer "F.Cu") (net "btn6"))
 (segment (start 54.0115 108.0395) (end 66.77792 95.27308) (width 0.2) (layer "F.Cu") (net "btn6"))
 (segment (start 54.0115 143.92275) (end 54.0115 108.0395) (width 0.2) (layer "F.Cu") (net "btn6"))
 (segment (start 17 112.73925) (end 17 82.051) (width 0.2) (layer "F.Cu") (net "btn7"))
 (segment (start 22.48 76.571) (end 44.15408 76.571) (width 0.2) (layer "F.Cu") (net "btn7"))
 (segment (start 17 82.051) (end 22.48 76.571) (width 0.2) (layer "F.Cu") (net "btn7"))
 (segment (start 44.6315 140.37075) (end 17 112.73925) (width 0.2) (layer "F.Cu") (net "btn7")))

